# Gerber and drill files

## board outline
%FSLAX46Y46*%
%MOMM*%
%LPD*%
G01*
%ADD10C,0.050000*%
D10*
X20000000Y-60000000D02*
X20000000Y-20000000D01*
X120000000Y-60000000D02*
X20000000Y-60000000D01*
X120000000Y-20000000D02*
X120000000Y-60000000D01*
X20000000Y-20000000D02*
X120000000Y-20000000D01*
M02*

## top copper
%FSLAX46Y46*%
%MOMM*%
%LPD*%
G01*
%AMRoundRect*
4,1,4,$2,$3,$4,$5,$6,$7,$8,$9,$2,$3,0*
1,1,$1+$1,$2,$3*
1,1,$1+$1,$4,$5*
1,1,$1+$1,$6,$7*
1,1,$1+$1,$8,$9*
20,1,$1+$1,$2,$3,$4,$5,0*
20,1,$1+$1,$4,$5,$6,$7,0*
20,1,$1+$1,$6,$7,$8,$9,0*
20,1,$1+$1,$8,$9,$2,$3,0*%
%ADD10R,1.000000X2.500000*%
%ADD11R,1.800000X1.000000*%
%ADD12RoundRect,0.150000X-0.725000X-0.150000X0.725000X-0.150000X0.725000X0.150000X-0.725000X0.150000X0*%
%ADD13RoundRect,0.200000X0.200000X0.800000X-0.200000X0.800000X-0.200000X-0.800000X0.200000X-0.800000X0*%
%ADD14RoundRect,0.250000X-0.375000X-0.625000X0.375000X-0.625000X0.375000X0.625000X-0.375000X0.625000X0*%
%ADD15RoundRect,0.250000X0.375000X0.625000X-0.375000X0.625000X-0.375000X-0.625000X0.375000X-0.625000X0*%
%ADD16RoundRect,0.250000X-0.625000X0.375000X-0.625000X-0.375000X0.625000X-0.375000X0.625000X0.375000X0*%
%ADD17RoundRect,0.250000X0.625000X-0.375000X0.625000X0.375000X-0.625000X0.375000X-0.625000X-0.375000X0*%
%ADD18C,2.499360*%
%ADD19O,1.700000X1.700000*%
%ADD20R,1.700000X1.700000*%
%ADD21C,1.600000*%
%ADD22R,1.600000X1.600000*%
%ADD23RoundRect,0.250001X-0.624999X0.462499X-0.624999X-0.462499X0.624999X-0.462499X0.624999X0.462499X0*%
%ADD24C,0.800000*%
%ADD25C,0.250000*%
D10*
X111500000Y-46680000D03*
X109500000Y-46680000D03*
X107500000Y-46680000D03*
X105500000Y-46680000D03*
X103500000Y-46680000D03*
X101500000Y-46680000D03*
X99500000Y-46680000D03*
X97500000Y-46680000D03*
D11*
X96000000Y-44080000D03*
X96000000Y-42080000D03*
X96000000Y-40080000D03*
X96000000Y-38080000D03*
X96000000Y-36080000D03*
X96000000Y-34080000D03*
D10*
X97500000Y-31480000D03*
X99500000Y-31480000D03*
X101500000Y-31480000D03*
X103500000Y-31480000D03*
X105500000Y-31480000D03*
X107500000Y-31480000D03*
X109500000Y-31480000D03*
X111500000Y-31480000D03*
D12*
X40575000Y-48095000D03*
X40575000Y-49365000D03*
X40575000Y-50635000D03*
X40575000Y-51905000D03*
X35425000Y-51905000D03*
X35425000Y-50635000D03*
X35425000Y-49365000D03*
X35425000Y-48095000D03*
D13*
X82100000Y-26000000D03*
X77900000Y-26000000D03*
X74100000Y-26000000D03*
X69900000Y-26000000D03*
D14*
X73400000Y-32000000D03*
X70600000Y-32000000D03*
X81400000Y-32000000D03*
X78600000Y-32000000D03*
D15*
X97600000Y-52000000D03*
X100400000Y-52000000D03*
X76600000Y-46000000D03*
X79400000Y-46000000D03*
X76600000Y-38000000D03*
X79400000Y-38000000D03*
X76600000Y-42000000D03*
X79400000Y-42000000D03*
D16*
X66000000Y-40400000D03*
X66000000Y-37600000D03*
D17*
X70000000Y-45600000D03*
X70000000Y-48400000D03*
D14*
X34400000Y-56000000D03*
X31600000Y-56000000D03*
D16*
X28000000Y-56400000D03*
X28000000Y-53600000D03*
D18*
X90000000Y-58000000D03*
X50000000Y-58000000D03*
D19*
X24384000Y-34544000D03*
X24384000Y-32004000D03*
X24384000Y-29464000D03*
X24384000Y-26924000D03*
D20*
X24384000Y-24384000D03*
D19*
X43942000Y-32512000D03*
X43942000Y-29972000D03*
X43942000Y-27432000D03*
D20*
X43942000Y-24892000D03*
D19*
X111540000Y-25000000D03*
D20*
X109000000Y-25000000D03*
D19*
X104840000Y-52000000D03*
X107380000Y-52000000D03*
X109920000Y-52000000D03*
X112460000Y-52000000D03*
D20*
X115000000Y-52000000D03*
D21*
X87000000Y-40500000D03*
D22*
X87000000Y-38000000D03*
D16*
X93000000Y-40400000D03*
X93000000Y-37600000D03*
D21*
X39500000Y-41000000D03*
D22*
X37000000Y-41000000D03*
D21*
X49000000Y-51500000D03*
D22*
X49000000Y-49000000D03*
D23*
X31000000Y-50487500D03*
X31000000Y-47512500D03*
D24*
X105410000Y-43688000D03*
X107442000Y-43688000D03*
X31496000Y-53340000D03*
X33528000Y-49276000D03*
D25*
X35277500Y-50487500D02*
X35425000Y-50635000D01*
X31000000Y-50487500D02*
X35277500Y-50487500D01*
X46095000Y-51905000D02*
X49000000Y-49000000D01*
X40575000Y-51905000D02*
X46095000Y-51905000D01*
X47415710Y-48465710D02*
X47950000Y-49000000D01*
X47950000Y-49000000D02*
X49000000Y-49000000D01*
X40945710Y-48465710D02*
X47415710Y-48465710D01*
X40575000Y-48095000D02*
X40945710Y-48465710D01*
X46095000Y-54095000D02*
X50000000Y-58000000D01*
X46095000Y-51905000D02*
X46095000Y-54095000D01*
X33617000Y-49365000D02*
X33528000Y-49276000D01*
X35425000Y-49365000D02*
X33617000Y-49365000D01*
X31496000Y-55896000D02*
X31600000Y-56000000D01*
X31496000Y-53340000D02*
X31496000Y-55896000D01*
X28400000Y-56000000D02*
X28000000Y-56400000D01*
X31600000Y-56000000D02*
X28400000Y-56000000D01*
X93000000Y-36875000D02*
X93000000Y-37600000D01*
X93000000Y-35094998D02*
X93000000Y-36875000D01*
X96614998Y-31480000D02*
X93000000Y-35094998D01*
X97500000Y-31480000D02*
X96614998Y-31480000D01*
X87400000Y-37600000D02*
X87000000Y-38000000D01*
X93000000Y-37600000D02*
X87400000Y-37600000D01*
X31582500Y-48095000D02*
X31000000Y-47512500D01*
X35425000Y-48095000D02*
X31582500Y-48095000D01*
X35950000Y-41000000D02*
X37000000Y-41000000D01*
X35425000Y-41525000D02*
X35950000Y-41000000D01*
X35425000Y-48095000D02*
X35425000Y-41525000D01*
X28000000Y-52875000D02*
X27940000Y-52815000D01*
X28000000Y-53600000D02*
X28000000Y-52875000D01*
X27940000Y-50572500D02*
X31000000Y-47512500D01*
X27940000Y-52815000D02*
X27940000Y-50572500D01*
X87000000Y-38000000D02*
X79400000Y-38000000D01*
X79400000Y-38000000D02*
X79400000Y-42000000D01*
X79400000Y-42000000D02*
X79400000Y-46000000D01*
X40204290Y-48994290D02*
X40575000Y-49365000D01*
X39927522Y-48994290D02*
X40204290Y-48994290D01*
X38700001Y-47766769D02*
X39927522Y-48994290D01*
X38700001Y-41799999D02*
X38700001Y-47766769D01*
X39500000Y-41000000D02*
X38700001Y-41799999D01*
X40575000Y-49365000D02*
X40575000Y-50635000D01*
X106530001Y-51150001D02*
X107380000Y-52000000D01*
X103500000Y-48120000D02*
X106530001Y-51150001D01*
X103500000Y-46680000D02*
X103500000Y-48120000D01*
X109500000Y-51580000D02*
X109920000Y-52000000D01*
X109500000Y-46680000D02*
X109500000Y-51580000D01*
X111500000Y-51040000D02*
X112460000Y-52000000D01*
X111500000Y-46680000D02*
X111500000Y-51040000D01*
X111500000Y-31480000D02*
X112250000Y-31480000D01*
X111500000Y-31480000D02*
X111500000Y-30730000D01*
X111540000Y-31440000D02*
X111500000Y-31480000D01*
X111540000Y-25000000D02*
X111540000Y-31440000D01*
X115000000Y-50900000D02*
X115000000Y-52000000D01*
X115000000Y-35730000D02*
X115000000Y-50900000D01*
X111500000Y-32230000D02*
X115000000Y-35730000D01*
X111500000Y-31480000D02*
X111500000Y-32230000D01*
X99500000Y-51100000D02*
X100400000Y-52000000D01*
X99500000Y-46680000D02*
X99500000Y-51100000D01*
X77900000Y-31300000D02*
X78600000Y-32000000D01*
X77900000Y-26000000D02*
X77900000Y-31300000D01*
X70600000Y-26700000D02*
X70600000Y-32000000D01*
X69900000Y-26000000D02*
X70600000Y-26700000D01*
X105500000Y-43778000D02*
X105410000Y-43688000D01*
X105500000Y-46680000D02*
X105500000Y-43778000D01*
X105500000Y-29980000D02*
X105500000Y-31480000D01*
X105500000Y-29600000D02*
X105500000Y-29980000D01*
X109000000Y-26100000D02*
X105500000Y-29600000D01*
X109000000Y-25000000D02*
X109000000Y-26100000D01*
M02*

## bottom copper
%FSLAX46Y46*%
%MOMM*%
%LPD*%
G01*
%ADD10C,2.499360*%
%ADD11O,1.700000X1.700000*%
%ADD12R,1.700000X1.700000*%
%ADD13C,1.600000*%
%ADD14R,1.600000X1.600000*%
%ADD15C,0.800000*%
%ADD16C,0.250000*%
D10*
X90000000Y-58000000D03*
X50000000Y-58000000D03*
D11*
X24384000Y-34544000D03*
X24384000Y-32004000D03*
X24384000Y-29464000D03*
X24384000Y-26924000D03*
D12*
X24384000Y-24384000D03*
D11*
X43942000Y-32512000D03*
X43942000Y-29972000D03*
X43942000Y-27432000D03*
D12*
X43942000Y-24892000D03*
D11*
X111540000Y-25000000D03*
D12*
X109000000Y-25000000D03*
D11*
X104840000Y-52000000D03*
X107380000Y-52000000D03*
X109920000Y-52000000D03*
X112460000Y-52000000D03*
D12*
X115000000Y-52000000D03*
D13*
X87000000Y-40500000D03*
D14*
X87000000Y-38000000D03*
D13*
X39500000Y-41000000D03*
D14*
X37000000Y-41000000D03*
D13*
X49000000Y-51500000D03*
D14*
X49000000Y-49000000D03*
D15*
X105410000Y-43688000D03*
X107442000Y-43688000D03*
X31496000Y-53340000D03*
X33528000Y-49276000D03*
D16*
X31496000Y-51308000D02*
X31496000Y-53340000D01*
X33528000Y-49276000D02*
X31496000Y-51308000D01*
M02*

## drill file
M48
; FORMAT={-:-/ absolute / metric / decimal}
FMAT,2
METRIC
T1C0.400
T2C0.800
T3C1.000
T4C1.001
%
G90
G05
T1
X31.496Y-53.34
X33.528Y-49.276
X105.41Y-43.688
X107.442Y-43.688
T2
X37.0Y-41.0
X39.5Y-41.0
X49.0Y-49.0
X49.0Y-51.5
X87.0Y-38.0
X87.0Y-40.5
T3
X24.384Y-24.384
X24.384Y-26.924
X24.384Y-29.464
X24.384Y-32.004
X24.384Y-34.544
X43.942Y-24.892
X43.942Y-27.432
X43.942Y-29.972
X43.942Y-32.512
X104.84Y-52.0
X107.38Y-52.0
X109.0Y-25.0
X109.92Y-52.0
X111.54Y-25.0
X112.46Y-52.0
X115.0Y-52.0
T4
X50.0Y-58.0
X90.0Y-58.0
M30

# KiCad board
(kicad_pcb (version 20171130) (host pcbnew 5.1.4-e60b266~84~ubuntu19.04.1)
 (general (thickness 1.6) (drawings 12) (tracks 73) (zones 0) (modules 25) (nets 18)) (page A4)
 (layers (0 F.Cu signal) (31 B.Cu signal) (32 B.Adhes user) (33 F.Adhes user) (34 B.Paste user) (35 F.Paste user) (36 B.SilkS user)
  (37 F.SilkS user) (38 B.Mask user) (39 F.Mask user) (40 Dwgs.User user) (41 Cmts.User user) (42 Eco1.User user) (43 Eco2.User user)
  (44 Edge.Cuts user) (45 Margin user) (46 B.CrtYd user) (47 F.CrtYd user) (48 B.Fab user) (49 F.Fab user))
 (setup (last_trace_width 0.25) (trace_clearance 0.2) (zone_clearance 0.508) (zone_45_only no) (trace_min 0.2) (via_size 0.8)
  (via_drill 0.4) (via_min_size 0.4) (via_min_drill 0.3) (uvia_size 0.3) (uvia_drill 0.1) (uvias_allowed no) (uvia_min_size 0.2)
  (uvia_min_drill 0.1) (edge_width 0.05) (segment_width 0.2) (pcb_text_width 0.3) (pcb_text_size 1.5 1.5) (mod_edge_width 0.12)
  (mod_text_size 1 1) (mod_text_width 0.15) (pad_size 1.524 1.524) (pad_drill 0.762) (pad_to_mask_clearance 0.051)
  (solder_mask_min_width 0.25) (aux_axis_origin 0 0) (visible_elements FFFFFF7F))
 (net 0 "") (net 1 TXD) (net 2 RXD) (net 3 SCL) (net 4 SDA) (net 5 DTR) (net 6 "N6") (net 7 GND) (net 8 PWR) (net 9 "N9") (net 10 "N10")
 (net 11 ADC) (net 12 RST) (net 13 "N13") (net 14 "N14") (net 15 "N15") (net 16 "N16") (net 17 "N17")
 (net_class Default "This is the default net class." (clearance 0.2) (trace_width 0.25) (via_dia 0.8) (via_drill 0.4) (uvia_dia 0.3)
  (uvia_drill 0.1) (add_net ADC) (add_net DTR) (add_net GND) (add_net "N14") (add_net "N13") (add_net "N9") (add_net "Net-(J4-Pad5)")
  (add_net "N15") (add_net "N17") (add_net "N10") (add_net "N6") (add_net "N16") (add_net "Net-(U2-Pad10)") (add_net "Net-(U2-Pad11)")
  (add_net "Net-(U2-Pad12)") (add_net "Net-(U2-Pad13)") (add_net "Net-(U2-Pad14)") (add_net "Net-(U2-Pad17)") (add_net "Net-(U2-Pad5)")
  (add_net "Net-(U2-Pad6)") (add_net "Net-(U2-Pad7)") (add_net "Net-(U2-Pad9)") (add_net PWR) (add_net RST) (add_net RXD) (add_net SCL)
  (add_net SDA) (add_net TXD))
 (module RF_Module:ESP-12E (layer F.Cu) (at 108 39.08 270)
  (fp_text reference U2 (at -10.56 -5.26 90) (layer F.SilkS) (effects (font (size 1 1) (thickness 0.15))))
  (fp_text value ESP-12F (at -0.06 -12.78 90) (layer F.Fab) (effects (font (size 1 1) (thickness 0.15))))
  (pad 22 smd rect (at 7.6 -3.5 270) (size 2.5 1) (layers F.Cu F.Paste F.Mask) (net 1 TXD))
  (pad 21 smd rect (at 7.6 -1.5 270) (size 2.5 1) (layers F.Cu F.Paste F.Mask) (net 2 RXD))
  (pad 20 smd rect (at 7.6 0.5 270) (size 2.5 1) (layers F.Cu F.Paste F.Mask) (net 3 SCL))
  (pad 19 smd rect (at 7.6 2.5 270) (size 2.5 1) (layers F.Cu F.Paste F.Mask) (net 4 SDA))
  (pad 18 smd rect (at 7.6 4.5 270) (size 2.5 1) (layers F.Cu F.Paste F.Mask) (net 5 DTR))
  (pad 17 smd rect (at 7.6 6.5 270) (size 2.5 1) (layers F.Cu F.Paste F.Mask))
  (pad 16 smd rect (at 7.6 8.5 270) (size 2.5 1) (layers F.Cu F.Paste F.Mask) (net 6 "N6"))
  (pad 15 smd rect (at 7.6 10.5 270) (size 2.5 1) (layers F.Cu F.Paste F.Mask) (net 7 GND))
  (pad 14 smd rect (at 5 12 270) (size 1 1.8) (layers F.Cu F.Paste F.Mask))
  (pad 13 smd rect (at 3 12 270) (size 1 1.8) (layers F.Cu F.Paste F.Mask))
  (pad 12 smd rect (at 1 12 270) (size 1 1.8) (layers F.Cu F.Paste F.Mask))
  (pad 11 smd rect (at -1 12 270) (size 1 1.8) (layers F.Cu F.Paste F.Mask))
  (pad 10 smd rect (at -3 12 270) (size 1 1.8) (layers F.Cu F.Paste F.Mask))
  (pad 9 smd rect (at -5 12 270) (size 1 1.8) (layers F.Cu F.Paste F.Mask))
  (pad 8 smd rect (at -7.6 10.5 270) (size 2.5 1) (layers F.Cu F.Paste F.Mask) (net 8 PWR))
  (pad 7 smd rect (at -7.6 8.5 270) (size 2.5 1) (layers F.Cu F.Paste F.Mask))
  (pad 6 smd rect (at -7.6 6.5 270) (size 2.5 1) (layers F.Cu F.Paste F.Mask))
  (pad 5 smd rect (at -7.6 4.5 270) (size 2.5 1) (layers F.Cu F.Paste F.Mask))
  (pad 4 smd rect (at -7.6 2.5 270) (size 2.5 1) (layers F.Cu F.Paste F.Mask) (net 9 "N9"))
  (pad 3 smd rect (at -7.6 0.5 270) (size 2.5 1) (layers F.Cu F.Paste F.Mask) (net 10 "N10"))
  (pad 2 smd rect (at -7.6 -1.5 270) (size 2.5 1) (layers F.Cu F.Paste F.Mask) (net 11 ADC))
  (pad 1 smd rect (at -7.6 -3.5 270) (size 2.5 1) (layers F.Cu F.Paste F.Mask) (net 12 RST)))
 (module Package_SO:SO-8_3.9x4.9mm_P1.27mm (layer F.Cu) (at 38 50)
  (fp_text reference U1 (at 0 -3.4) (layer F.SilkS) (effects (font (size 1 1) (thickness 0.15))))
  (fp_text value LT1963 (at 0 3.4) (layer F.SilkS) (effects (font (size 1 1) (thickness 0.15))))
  (pad 8 smd roundrect (at 2.575 -1.905) (size 1.75 0.6) (layers F.Cu F.Paste F.Mask) (roundrect_rratio 0.25) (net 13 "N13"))
  (pad 7 smd roundrect (at 2.575 -0.635) (size 1.75 0.6) (layers F.Cu F.Paste F.Mask) (roundrect_rratio 0.25) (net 7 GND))
  (pad 6 smd roundrect (at 2.575 0.635) (size 1.75 0.6) (layers F.Cu F.Paste F.Mask) (roundrect_rratio 0.25) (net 7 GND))
  (pad 5 smd roundrect (at 2.575 1.905) (size 1.75 0.6) (layers F.Cu F.Paste F.Mask) (roundrect_rratio 0.25) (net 13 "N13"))
  (pad 4 smd roundrect (at -2.575 1.905) (size 1.75 0.6) (layers F.Cu F.Paste F.Mask) (roundrect_rratio 0.25) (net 7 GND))
  (pad 3 smd roundrect (at -2.575 0.635) (size 1.75 0.6) (layers F.Cu F.Paste F.Mask) (roundrect_rratio 0.25) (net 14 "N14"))
  (pad 2 smd roundrect (at -2.575 -0.635) (size 1.75 0.6) (layers F.Cu F.Paste F.Mask) (roundrect_rratio 0.25) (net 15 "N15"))
  (pad 1 smd roundrect (at -2.575 -1.905) (size 1.75 0.6) (layers F.Cu F.Paste F.Mask) (roundrect_rratio 0.25) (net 8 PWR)))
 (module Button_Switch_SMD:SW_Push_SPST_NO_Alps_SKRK (layer F.Cu) (at 80 26 180)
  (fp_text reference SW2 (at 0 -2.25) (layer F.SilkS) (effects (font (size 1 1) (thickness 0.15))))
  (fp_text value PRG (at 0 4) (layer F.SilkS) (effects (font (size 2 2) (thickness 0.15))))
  (pad 1 smd roundrect (at -2.1 0 180) (size 0.8 2) (layers F.Cu F.Paste F.Mask) (roundrect_rratio 0.25) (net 5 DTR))
  (pad 2 smd roundrect (at 2.1 0 180) (size 0.8 2) (layers F.Cu F.Paste F.Mask) (roundrect_rratio 0.25) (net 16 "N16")))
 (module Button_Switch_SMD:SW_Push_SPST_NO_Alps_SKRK (layer F.Cu) (at 72 26 180)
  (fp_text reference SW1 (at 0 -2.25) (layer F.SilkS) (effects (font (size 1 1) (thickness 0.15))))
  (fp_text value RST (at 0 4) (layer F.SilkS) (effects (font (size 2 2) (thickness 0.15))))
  (pad 1 smd roundrect (at -2.1 0 180) (size 0.8 2) (layers F.Cu F.Paste F.Mask) (roundrect_rratio 0.25) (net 12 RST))
  (pad 2 smd roundrect (at 2.1 0 180) (size 0.8 2) (layers F.Cu F.Paste F.Mask) (roundrect_rratio 0.25) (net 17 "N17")))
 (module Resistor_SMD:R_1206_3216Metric (layer F.Cu) (at 72 32)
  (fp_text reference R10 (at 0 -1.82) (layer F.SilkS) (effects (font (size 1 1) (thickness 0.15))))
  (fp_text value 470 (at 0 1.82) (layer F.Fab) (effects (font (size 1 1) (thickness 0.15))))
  (pad 2 smd roundrect (at 1.4 0) (size 1.25 1.75) (layers F.Cu F.Paste F.Mask) (roundrect_rratio 0.2) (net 7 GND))
  (pad 1 smd roundrect (at -1.4 0) (size 1.25 1.75) (layers F.Cu F.Paste F.Mask) (roundrect_rratio 0.2) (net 17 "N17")))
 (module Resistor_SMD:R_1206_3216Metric (layer F.Cu) (at 80 32)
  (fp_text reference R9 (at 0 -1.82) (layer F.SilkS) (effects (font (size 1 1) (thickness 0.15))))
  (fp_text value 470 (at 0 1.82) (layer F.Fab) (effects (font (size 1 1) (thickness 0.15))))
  (pad 2 smd roundrect (at 1.4 0) (size 1.25 1.75) (layers F.Cu F.Paste F.Mask) (roundrect_rratio 0.2) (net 7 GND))
  (pad 1 smd roundrect (at -1.4 0) (size 1.25 1.75) (layers F.Cu F.Paste F.Mask) (roundrect_rratio 0.2) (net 16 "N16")))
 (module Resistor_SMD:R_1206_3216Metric (layer F.Cu) (at 99 52 180)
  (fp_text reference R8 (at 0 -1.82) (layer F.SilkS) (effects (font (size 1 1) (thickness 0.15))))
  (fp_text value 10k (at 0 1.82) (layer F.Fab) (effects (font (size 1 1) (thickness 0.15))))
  (pad 2 smd roundrect (at 1.4 0 180) (size 1.25 1.75) (layers F.Cu F.Paste F.Mask) (roundrect_rratio 0.2) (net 7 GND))
  (pad 1 smd roundrect (at -1.4 0 180) (size 1.25 1.75) (layers F.Cu F.Paste F.Mask) (roundrect_rratio 0.2) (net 6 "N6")))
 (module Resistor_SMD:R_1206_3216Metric (layer F.Cu) (at 78 46 180)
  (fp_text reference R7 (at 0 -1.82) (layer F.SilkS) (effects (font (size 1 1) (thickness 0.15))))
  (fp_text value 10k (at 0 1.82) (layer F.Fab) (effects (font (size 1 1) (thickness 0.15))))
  (pad 2 smd roundrect (at 1.4 0 180) (size 1.25 1.75) (layers F.Cu F.Paste F.Mask) (roundrect_rratio 0.2) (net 5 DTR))
  (pad 1 smd roundrect (at -1.4 0 180) (size 1.25 1.75) (layers F.Cu F.Paste F.Mask) (roundrect_rratio 0.2) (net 8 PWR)))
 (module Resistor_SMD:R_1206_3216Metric (layer F.Cu) (at 78 38 180)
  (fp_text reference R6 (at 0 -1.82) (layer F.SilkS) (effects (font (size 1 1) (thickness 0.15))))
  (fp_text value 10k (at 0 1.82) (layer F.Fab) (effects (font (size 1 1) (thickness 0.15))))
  (pad 2 smd roundrect (at 1.4 0 180) (size 1.25 1.75) (layers F.Cu F.Paste F.Mask) (roundrect_rratio 0.2) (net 12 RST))
  (pad 1 smd roundrect (at -1.4 0 180) (size 1.25 1.75) (layers F.Cu F.Paste F.Mask) (roundrect_rratio 0.2) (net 8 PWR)))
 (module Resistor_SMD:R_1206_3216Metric (layer F.Cu) (at 78 42 180)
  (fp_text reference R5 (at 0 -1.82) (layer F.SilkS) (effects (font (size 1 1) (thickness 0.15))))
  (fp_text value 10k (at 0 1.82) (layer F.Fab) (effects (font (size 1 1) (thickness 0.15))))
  (pad 2 smd roundrect (at 1.4 0 180) (size 1.25 1.75) (layers F.Cu F.Paste F.Mask) (roundrect_rratio 0.2) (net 10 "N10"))
  (pad 1 smd roundrect (at -1.4 0 180) (size 1.25 1.75) (layers F.Cu F.Paste F.Mask) (roundrect_rratio 0.2) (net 8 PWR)))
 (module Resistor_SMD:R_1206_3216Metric (layer F.Cu) (at 66 39 270)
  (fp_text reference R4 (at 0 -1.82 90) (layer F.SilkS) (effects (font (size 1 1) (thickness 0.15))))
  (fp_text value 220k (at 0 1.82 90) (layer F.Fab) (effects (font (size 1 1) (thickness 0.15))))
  (pad 2 smd roundrect (at 1.4 0 270) (size 1.25 1.75) (layers F.Cu F.Paste F.Mask) (roundrect_rratio 0.2) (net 7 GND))
  (pad 1 smd roundrect (at -1.4 0 270) (size 1.25 1.75) (layers F.Cu F.Paste F.Mask) (roundrect_rratio 0.2) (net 11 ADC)))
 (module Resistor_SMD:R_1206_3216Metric (layer F.Cu) (at 70 47 90)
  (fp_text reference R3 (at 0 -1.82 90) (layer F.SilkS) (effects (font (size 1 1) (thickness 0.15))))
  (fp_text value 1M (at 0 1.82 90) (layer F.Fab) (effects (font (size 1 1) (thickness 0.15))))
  (pad 2 smd roundrect (at 1.4 0 90) (size 1.25 1.75) (layers F.Cu F.Paste F.Mask) (roundrect_rratio 0.2) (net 11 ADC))
  (pad 1 smd roundrect (at -1.4 0 90) (size 1.25 1.75) (layers F.Cu F.Paste F.Mask) (roundrect_rratio 0.2) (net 13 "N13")))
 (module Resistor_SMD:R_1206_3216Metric (layer F.Cu) (at 33 56)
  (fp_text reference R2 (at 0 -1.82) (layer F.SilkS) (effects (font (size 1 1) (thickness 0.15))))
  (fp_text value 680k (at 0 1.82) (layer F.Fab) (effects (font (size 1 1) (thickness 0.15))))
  (pad 2 smd roundrect (at 1.4 0) (size 1.25 1.75) (layers F.Cu F.Paste F.Mask) (roundrect_rratio 0.2) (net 7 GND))
  (pad 1 smd roundrect (at -1.4 0) (size 1.25 1.75) (layers F.Cu F.Paste F.Mask) (roundrect_rratio 0.2) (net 15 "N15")))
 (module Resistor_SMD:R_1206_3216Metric (layer F.Cu) (at 28 55 270)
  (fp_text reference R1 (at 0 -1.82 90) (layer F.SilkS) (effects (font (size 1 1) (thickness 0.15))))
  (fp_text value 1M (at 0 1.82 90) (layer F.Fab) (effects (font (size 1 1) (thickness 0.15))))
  (pad 2 smd roundrect (at 1.4 0 270) (size 1.25 1.75) (layers F.Cu F.Paste F.Mask) (roundrect_rratio 0.2) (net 15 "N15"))
  (pad 1 smd roundrect (at -1.4 0 270) (size 1.25 1.75) (layers F.Cu F.Paste F.Mask) (roundrect_rratio 0.2) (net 8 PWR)))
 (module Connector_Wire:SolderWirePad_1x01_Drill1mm (layer F.Cu) (at 90 58)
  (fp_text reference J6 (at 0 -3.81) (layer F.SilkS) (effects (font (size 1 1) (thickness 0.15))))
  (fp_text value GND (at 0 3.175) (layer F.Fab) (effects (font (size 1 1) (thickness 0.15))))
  (pad 1 thru_hole circle (at 0 0) (size 2.49936 2.49936) (drill 1.00076) (layers *.Cu *.Mask) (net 7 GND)))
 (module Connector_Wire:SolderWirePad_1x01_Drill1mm (layer F.Cu) (at 50 58)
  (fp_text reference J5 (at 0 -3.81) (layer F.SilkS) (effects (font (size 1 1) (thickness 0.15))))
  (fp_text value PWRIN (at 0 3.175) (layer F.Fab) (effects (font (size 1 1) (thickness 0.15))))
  (pad 1 thru_hole circle (at 0 0) (size 2.49936 2.49936) (drill 1.00076) (layers *.Cu *.Mask) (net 13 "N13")))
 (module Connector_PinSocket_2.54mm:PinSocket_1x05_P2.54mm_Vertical (layer F.Cu) (at 24.384 24.384)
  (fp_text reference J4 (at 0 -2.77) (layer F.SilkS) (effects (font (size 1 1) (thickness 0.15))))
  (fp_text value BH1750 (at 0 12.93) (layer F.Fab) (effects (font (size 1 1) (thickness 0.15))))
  (pad 5 thru_hole oval (at 0 10.16) (size 1.7 1.7) (drill 1) (layers *.Cu *.Mask))
  (pad 4 thru_hole oval (at 0 7.62) (size 1.7 1.7) (drill 1) (layers *.Cu *.Mask) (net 4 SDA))
  (pad 3 thru_hole oval (at 0 5.08) (size 1.7 1.7) (drill 1) (layers *.Cu *.Mask) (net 3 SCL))
  (pad 2 thru_hole oval (at 0 2.54) (size 1.7 1.7) (drill 1) (layers *.Cu *.Mask) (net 7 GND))
  (pad 1 thru_hole rect (at 0 0) (size 1.7 1.7) (drill 1) (layers *.Cu *.Mask) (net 8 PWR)))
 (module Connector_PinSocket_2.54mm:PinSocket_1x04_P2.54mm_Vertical (layer F.Cu) (at 43.942 24.892)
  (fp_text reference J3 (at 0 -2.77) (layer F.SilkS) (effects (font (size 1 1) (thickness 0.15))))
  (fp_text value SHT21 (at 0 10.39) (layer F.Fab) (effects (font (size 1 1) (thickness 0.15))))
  (pad 4 thru_hole oval (at 0 7.62) (size 1.7 1.7) (drill 1) (layers *.Cu *.Mask) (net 4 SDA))
  (pad 3 thru_hole oval (at 0 5.08) (size 1.7 1.7) (drill 1) (layers *.Cu *.Mask) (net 3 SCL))
  (pad 2 thru_hole oval (at 0 2.54) (size 1.7 1.7) (drill 1) (layers *.Cu *.Mask) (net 7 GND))
  (pad 1 thru_hole rect (at 0 0) (size 1.7 1.7) (drill 1) (layers *.Cu *.Mask) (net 8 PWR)))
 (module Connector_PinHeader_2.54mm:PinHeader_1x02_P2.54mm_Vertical (layer F.Cu) (at 109 25 90)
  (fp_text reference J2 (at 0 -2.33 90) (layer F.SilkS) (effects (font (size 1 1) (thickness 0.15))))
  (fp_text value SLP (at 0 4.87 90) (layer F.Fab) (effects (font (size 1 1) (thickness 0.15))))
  (pad 2 thru_hole oval (at 0 2.54 90) (size 1.7 1.7) (drill 1) (layers *.Cu *.Mask) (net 12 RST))
  (pad 1 thru_hole rect (at 0 0 90) (size 1.7 1.7) (drill 1) (layers *.Cu *.Mask) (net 9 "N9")))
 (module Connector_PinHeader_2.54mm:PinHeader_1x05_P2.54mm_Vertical (layer F.Cu) (at 115 52 270)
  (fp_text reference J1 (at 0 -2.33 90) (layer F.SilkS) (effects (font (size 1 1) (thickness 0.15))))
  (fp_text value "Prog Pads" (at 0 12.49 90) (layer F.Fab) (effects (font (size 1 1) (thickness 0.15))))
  (pad 5 thru_hole oval (at 0 10.16 270) (size 1.7 1.7) (drill 1) (layers *.Cu *.Mask) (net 7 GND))
  (pad 4 thru_hole oval (at 0 7.62 270) (size 1.7 1.7) (drill 1) (layers *.Cu *.Mask) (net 5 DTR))
  (pad 3 thru_hole oval (at 0 5.08 270) (size 1.7 1.7) (drill 1) (layers *.Cu *.Mask) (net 2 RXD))
  (pad 2 thru_hole oval (at 0 2.54 270) (size 1.7 1.7) (drill 1) (layers *.Cu *.Mask) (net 1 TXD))
  (pad 1 thru_hole rect (at 0 0 270) (size 1.7 1.7) (drill 1) (layers *.Cu *.Mask) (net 12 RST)))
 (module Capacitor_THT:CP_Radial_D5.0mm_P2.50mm (layer F.Cu) (at 87 38 270)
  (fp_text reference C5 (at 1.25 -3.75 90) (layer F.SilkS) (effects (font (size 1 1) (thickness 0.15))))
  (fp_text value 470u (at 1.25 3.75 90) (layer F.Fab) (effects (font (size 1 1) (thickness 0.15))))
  (pad 2 thru_hole circle (at 2.5 0 270) (size 1.6 1.6) (drill 0.8) (layers *.Cu *.Mask) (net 7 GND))
  (pad 1 thru_hole rect (at 0 0 270) (size 1.6 1.6) (drill 0.8) (layers *.Cu *.Mask) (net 8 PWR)))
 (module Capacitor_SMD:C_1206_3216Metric (layer F.Cu) (at 93 39 270)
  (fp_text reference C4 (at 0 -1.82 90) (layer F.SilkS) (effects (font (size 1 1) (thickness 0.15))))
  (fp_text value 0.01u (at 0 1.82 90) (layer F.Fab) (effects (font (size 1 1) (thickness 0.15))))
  (pad 2 smd roundrect (at 1.4 0 270) (size 1.25 1.75) (layers F.Cu F.Paste F.Mask) (roundrect_rratio 0.2) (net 7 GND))
  (pad 1 smd roundrect (at -1.4 0 270) (size 1.25 1.75) (layers F.Cu F.Paste F.Mask) (roundrect_rratio 0.2) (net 8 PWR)))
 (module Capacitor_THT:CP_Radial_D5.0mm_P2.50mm (layer F.Cu) (at 37 41)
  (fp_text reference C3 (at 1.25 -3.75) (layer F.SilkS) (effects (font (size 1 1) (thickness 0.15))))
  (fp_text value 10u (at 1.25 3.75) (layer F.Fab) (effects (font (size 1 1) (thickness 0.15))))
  (pad 2 thru_hole circle (at 2.5 0) (size 1.6 1.6) (drill 0.8) (layers *.Cu *.Mask) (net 7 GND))
  (pad 1 thru_hole rect (at 0 0) (size 1.6 1.6) (drill 0.8) (layers *.Cu *.Mask) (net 8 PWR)))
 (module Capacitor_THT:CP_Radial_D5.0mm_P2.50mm (layer F.Cu) (at 49 49 270)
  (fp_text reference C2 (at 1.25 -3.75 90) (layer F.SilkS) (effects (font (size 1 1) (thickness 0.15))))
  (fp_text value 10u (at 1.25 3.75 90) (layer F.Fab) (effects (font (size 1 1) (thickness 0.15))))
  (pad 2 thru_hole circle (at 2.5 0 270) (size 1.6 1.6) (drill 0.8) (layers *.Cu *.Mask) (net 7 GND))
  (pad 1 thru_hole rect (at 0 0 270) (size 1.6 1.6) (drill 0.8) (layers *.Cu *.Mask) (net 13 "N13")))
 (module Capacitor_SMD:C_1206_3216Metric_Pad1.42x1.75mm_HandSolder (layer F.Cu) (at 31 49 270)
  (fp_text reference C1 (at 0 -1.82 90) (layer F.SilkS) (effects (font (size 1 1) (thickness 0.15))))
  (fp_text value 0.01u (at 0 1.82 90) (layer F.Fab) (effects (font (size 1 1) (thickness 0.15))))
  (pad 2 smd roundrect (at 1.4875 0 270) (size 1.425 1.75) (layers F.Cu F.Paste F.Mask) (roundrect_rratio 0.175439) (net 14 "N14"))
  (pad 1 smd roundrect (at -1.4875 0 270) (size 1.425 1.75) (layers F.Cu F.Paste F.Mask) (roundrect_rratio 0.175439) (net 8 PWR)))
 (gr_line (start 20 60) (end 20 20) (layer Edge.Cuts) (width 0.05))
 (gr_line (start 120 60) (end 20 60) (layer Edge.Cuts) (width 0.05))
 (gr_line (start 120 20) (end 120 60) (layer Edge.Cuts) (width 0.05))
 (gr_line (start 20 20) (end 120 20) (layer Edge.Cuts) (width 0.05))
 (via (at 105.41 43.688) (size 0.8) (drill 0.4) (layers F.Cu B.Cu) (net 4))
 (via (at 107.442 43.688) (size 0.8) (drill 0.4) (layers F.Cu B.Cu) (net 3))
 (via (at 31.496 53.34) (size 0.8) (drill 0.4) (layers F.Cu B.Cu) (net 15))
 (via (at 33.528 49.276) (size 0.8) (drill 0.4) (layers F.Cu B.Cu) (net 15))
 (segment (start 35.2775 50.4875) (end 35.425 50.635) (width 0.25) (layer F.Cu) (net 14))
 (segment (start 31 50.4875) (end 35.2775 50.4875) (width 0.25) (layer F.Cu) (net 14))
 (segment (start 46.095 51.905) (end 49 49) (width 0.25) (layer F.Cu) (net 13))
 (segment (start 40.575 51.905) (end 46.095 51.905) (width 0.25) (layer F.Cu) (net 13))
 (segment (start 47.41571 48.46571) (end 47.95 49) (width 0.25) (layer F.Cu) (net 13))
 (segment (start 47.95 49) (end 49 49) (width 0.25) (layer F.Cu) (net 13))
 (segment (start 40.94571 48.46571) (end 47.41571 48.46571) (width 0.25) (layer F.Cu) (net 13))
 (segment (start 40.575 48.095) (end 40.94571 48.46571) (width 0.25) (layer F.Cu) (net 13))
 (segment (start 46.095 54.095) (end 50 58) (width 0.25) (layer F.Cu) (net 13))
 (segment (start 46.095 51.905) (end 46.095 54.095) (width 0.25) (layer F.Cu) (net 13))
 (segment (start 33.617 49.365) (end 33.528 49.276) (width 0.25) (layer F.Cu) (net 15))
 (segment (start 35.425 49.365) (end 33.617 49.365) (width 0.25) (layer F.Cu) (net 15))
 (segment (start 31.496 51.308) (end 31.496 53.34) (width 0.25) (layer B.Cu) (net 15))
 (segment (start 33.528 49.276) (end 31.496 51.308) (width 0.25) (layer B.Cu) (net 15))
 (segment (start 31.496 55.896) (end 31.6 56) (width 0.25) (layer F.Cu) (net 15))
 (segment (start 31.496 53.34) (end 31.496 55.896) (width 0.25) (layer F.Cu) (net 15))
 (segment (start 28.4 56) (end 28 56.4) (width 0.25) (layer F.Cu) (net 15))
 (segment (start 31.6 56) (end 28.4 56) (width 0.25) (layer F.Cu) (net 15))
 (segment (start 93 36.875) (end 93 37.6) (width 0.25) (layer F.Cu) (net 8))
 (segment (start 93 35.094998) (end 93 36.875) (width 0.25) (layer F.Cu) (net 8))
 (segment (start 96.614998 31.48) (end 93 35.094998) (width 0.25) (layer F.Cu) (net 8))
 (segment (start 97.5 31.48) (end 96.614998 31.48) (width 0.25) (layer F.Cu) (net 8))
 (segment (start 87.4 37.6) (end 87 38) (width 0.25) (layer F.Cu) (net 8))
 (segment (start 93 37.6) (end 87.4 37.6) (width 0.25) (layer F.Cu) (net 8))
 (segment (start 31.5825 48.095) (end 31 47.5125) (width 0.25) (layer F.Cu) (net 8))
 (segment (start 35.425 48.095) (end 31.5825 48.095) (width 0.25) (layer F.Cu) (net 8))
 (segment (start 35.95 41) (end 37 41) (width 0.25) (layer F.Cu) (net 8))
 (segment (start 35.425 41.525) (end 35.95 41) (width 0.25) (layer F.Cu) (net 8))
 (segment (start 35.425 48.095) (end 35.425 41.525) (width 0.25) (layer F.Cu) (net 8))
 (segment (start 28 52.875) (end 27.94 52.815) (width 0.25) (layer F.Cu) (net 8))
 (segment (start 28 53.6) (end 28 52.875) (width 0.25) (layer F.Cu) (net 8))
 (segment (start 27.94 50.5725) (end 31 47.5125) (width 0.25) (layer F.Cu) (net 8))
 (segment (start 27.94 52.815) (end 27.94 50.5725) (width 0.25) (layer F.Cu) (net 8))
 (segment (start 87 38) (end 79.4 38) (width 0.25) (layer F.Cu) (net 8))
 (segment (start 79.4 38) (end 79.4 42) (width 0.25) (layer F.Cu) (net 8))
 (segment (start 79.4 42) (end 79.4 46) (width 0.25) (layer F.Cu) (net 8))
 (segment (start 40.20429 48.99429) (end 40.575 49.365) (width 0.25) (layer F.Cu) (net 7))
 (segment (start 39.927522 48.99429) (end 40.20429 48.99429) (width 0.25) (layer F.Cu) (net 7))
 (segment (start 38.700001 47.766769) (end 39.927522 48.99429) (width 0.25) (layer F.Cu) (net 7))
 (segment (start 38.700001 41.799999) (end 38.700001 47.766769) (width 0.25) (layer F.Cu) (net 7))
 (segment (start 39.5 41) (end 38.700001 41.799999) (width 0.25) (layer F.Cu) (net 7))
 (segment (start 40.575 49.365) (end 40.575 50.635) (width 0.25) (layer F.Cu) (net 7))
 (segment (start 106.530001 51.150001) (end 107.38 52) (width 0.25) (layer F.Cu) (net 5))
 (segment (start 103.5 48.12) (end 106.530001 51.150001) (width 0.25) (layer F.Cu) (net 5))
 (segment (start 103.5 46.68) (end 103.5 48.12) (width 0.25) (layer F.Cu) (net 5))
 (segment (start 109.5 51.58) (end 109.92 52) (width 0.25) (layer F.Cu) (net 2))
 (segment (start 109.5 46.68) (end 109.5 51.58) (width 0.25) (layer F.Cu) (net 2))
 (segment (start 111.5 51.04) (end 112.46 52) (width 0.25) (layer F.Cu) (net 1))
 (segment (start 111.5 46.68) (end 111.5 51.04) (width 0.25) (layer F.Cu) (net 1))
 (segment (start 111.5 31.48) (end 112.25 31.48) (width 0.25) (layer F.Cu) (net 12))
 (segment (start 111.5 31.48) (end 111.5 30.73) (width 0.25) (layer F.Cu) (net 12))
 (segment (start 111.54 31.44) (end 111.5 31.48) (width 0.25) (layer F.Cu) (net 12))
 (segment (start 111.54 25) (end 111.54 31.44) (width 0.25) (layer F.Cu) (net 12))
 (segment (start 115 50.9) (end 115 52) (width 0.25) (layer F.Cu) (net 12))
 (segment (start 115 35.73) (end 115 50.9) (width 0.25) (layer F.Cu) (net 12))
 (segment (start 111.5 32.23) (end 115 35.73) (width 0.25) (layer F.Cu) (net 12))
 (segment (start 111.5 31.48) (end 111.5 32.23) (width 0.25) (layer F.Cu) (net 12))
 (segment (start 99.5 51.1) (end 100.4 52) (width 0.25) (layer F.Cu) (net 6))
 (segment (start 99.5 46.68) (end 99.5 51.1) (width 0.25) (layer F.Cu) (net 6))
 (segment (start 77.9 31.3) (end 78.6 32) (width 0.25) (layer F.Cu) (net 16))
 (segment (start 77.9 26) (end 77.9 31.3) (width 0.25) (layer F.Cu) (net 16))
 (segment (start 70.6 26.7) (end 70.6 32) (width 0.25) (layer F.Cu) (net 17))
 (segment (start 69.9 26) (end 70.6 26.7) (width 0.25) (layer F.Cu) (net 17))
 (segment (start 105.5 43.778) (end 105.41 43.688) (width 0.25) (layer F.Cu) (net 4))
 (segment (start 105.5 46.68) (end 105.5 43.778) (width 0.25) (layer F.Cu) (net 4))
 (segment (start 105.5 29.98) (end 105.5 31.48) (width 0.25) (layer F.Cu) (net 9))
 (segment (start 105.5 29.6) (end 105.5 29.98) (width 0.25) (layer F.Cu) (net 9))
 (segment (start 109 26.1) (end 105.5 29.6) (width 0.25) (layer F.Cu) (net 9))
 (segment (start 109 25) (end 109 26.1) (width 0.25) (layer F.Cu) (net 9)))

